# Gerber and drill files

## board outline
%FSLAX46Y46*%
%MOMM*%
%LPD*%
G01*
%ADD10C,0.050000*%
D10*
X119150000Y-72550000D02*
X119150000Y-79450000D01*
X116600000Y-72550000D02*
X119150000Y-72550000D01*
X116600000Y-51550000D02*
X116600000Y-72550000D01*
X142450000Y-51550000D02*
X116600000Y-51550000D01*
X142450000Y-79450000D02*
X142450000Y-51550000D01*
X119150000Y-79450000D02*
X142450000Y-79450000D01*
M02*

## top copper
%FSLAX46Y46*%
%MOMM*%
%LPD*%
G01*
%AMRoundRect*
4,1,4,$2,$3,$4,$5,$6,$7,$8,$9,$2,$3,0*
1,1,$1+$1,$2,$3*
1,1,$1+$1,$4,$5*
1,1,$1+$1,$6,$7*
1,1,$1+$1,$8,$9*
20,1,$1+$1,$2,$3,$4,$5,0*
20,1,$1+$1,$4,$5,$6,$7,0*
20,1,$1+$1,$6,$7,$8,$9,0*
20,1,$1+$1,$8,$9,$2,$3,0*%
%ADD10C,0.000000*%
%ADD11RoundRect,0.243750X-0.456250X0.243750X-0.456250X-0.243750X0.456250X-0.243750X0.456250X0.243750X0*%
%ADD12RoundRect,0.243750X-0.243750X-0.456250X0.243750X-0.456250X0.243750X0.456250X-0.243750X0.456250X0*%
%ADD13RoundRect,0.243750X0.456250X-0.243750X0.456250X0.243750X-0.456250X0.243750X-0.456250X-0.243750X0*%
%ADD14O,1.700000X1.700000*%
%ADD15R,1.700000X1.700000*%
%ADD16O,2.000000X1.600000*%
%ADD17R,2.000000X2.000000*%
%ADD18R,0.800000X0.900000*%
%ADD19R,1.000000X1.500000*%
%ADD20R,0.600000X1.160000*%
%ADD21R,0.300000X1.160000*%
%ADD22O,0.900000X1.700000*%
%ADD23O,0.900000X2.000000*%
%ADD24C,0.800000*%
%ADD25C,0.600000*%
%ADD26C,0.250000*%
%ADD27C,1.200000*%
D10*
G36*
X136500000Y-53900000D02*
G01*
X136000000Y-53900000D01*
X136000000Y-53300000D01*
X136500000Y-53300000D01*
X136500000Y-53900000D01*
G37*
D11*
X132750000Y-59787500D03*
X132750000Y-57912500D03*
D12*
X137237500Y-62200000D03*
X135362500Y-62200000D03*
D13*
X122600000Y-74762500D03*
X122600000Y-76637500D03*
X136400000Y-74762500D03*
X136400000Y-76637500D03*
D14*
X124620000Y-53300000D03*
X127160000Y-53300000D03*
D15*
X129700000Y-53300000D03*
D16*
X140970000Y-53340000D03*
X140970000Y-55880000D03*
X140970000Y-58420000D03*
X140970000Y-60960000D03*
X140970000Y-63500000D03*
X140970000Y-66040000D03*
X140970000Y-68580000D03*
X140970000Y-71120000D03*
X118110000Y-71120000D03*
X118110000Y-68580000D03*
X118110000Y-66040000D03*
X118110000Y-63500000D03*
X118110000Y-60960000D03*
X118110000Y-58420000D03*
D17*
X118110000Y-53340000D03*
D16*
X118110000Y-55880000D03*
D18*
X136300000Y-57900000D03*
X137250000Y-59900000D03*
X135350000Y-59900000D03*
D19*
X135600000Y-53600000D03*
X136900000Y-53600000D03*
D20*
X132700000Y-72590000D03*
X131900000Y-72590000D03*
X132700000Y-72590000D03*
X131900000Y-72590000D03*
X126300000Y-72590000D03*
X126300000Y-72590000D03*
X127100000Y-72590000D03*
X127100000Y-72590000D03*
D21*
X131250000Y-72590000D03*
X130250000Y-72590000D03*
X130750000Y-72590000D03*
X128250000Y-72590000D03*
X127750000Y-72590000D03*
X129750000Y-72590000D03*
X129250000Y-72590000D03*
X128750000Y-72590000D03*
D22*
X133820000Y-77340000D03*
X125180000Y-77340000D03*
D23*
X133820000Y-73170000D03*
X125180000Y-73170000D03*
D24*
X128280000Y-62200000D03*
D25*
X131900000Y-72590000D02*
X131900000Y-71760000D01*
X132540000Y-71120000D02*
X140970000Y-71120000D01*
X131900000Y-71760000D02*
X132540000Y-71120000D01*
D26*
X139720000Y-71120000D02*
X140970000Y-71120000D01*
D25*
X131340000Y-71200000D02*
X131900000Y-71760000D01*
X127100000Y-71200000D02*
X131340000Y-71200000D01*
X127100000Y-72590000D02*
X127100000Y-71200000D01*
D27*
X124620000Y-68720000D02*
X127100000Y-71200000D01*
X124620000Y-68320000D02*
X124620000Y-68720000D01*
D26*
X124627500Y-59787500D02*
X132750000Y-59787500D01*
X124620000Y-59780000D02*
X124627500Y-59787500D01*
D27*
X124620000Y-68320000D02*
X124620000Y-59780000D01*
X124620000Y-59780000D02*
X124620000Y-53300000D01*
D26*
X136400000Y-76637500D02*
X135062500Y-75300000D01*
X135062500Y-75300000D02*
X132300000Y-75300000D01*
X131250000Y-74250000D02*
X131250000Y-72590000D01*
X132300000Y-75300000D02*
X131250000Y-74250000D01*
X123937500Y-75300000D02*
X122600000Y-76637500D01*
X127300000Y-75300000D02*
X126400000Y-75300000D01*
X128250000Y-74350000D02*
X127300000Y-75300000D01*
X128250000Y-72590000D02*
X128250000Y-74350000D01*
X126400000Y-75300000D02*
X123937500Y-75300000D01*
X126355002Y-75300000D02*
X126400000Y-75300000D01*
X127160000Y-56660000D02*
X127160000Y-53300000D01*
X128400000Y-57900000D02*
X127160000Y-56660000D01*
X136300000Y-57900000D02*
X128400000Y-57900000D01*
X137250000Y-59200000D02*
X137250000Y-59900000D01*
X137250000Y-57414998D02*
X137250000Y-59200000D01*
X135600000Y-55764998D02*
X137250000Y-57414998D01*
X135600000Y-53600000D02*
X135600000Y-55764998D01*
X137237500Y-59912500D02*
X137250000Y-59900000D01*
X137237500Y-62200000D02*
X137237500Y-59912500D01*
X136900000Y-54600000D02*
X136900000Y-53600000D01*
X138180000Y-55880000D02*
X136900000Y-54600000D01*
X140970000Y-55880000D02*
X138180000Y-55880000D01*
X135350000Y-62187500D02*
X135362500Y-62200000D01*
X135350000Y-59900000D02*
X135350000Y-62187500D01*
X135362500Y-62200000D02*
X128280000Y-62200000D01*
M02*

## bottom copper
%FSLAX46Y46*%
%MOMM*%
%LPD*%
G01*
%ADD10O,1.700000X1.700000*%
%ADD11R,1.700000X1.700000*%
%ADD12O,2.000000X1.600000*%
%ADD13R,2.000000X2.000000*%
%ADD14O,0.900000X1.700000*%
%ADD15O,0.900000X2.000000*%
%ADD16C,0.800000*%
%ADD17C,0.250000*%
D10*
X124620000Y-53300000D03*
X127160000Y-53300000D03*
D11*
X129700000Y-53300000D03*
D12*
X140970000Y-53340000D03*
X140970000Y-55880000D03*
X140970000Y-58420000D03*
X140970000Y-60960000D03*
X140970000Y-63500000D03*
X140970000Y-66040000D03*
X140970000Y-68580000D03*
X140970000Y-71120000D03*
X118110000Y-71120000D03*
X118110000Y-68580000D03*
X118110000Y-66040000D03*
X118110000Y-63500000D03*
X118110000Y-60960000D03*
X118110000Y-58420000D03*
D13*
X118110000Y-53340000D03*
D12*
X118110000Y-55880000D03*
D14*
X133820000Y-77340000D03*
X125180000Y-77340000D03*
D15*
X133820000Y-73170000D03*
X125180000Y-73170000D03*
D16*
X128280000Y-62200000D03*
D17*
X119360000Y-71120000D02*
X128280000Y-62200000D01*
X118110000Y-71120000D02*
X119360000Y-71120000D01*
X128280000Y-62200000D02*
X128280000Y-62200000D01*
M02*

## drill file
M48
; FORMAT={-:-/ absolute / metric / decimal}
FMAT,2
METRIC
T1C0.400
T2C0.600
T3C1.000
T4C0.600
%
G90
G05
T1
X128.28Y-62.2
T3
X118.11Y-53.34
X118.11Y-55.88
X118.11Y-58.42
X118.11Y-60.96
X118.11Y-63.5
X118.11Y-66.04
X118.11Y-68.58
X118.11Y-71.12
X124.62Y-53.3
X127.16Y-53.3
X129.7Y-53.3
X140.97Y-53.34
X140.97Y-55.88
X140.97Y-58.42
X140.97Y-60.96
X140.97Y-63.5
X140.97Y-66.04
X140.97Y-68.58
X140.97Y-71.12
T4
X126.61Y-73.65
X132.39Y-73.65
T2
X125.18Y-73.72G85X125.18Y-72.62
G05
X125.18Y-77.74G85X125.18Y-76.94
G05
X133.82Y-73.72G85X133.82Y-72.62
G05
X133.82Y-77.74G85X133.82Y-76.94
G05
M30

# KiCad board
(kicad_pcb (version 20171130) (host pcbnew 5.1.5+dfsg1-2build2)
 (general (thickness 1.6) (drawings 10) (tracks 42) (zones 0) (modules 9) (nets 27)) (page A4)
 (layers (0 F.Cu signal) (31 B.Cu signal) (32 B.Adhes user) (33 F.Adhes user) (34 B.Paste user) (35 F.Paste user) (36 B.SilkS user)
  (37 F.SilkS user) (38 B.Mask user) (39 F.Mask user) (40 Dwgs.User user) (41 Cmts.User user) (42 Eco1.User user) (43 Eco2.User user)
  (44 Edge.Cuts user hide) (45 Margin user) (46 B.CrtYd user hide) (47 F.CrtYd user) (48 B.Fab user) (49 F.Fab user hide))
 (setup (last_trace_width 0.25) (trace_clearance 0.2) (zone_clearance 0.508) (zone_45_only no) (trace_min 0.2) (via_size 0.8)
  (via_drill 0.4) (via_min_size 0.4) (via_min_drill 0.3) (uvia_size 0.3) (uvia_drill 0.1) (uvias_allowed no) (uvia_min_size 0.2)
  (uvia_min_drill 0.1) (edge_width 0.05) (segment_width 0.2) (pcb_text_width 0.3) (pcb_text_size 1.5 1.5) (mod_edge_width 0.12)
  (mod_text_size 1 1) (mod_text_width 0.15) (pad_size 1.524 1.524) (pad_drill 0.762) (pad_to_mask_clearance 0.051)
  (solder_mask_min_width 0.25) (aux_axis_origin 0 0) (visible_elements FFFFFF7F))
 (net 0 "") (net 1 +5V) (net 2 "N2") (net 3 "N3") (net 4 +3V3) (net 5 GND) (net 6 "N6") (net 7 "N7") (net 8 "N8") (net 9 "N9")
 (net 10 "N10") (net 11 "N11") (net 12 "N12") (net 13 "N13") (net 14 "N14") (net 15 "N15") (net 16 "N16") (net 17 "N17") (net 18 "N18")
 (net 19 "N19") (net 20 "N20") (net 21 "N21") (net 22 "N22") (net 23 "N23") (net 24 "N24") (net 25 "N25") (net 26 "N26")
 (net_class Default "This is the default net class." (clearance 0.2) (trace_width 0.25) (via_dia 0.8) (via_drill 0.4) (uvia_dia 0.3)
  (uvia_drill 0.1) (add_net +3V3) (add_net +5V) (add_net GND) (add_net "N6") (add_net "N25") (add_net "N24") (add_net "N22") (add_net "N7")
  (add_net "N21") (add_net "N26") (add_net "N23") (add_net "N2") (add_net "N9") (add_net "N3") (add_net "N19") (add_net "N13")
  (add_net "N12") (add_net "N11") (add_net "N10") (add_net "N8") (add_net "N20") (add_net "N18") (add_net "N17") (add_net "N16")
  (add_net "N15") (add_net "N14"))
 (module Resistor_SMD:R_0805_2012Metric (layer F.Cu) (at 132.75 58.85 270)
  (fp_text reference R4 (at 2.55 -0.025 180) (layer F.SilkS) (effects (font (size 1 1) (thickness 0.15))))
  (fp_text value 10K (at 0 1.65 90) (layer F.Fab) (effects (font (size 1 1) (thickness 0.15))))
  (pad 2 smd roundrect (at 0.9375 0 270) (size 0.975 1.4) (layers F.Cu F.Paste F.Mask) (roundrect_rratio 0.25) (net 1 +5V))
  (pad 1 smd roundrect (at -0.9375 0 270) (size 0.975 1.4) (layers F.Cu F.Paste F.Mask) (roundrect_rratio 0.25) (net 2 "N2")))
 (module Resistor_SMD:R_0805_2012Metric (layer F.Cu) (at 136.3 62.2)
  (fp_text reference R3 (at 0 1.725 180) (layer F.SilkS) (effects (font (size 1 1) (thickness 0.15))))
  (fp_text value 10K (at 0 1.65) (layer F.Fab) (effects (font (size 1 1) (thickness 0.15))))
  (pad 2 smd roundrect (at 0.9375 0) (size 0.975 1.4) (layers F.Cu F.Paste F.Mask) (roundrect_rratio 0.25) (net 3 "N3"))
  (pad 1 smd roundrect (at -0.9375 0) (size 0.975 1.4) (layers F.Cu F.Paste F.Mask) (roundrect_rratio 0.25) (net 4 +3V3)))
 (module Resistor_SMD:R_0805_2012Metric (layer F.Cu) (at 122.6 75.7 90)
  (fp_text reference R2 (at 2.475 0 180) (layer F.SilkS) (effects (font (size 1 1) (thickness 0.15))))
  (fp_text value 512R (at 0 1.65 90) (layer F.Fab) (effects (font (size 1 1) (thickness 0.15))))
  (pad 2 smd roundrect (at 0.9375 0 90) (size 0.975 1.4) (layers F.Cu F.Paste F.Mask) (roundrect_rratio 0.25) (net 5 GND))
  (pad 1 smd roundrect (at -0.9375 0 90) (size 0.975 1.4) (layers F.Cu F.Paste F.Mask) (roundrect_rratio 0.25) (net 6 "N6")))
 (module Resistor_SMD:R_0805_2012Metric (layer F.Cu) (at 136.4 75.7 90)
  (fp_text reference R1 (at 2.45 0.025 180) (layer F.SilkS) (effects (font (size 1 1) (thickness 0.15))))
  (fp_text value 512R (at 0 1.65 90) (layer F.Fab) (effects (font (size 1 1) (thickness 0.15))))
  (pad 2 smd roundrect (at 0.9375 0 90) (size 0.975 1.4) (layers F.Cu F.Paste F.Mask) (roundrect_rratio 0.25) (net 5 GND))
  (pad 1 smd roundrect (at -0.9375 0 90) (size 0.975 1.4) (layers F.Cu F.Paste F.Mask) (roundrect_rratio 0.25) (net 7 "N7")))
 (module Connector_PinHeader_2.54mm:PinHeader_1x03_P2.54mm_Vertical (layer F.Cu) (at 129.7 53.3 270)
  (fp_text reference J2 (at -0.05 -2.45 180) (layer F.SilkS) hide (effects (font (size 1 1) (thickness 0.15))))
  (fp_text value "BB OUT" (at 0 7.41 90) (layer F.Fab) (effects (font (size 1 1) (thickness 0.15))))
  (pad 3 thru_hole oval (at 0 5.08 270) (size 1.7 1.7) (drill 1) (layers *.Cu *.Mask) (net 1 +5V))
  (pad 2 thru_hole oval (at 0 2.54 270) (size 1.7 1.7) (drill 1) (layers *.Cu *.Mask) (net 2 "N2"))
  (pad 1 thru_hole rect (at 0 0 270) (size 1.7 1.7) (drill 1) (layers *.Cu *.Mask) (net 5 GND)))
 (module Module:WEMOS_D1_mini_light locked (layer F.Cu) (at 118.11 53.34)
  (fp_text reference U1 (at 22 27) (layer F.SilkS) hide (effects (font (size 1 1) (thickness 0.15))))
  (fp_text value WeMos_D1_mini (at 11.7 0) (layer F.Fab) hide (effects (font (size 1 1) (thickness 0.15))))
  (pad 16 thru_hole oval (at 22.86 0) (size 2 1.6) (drill 1) (layers *.Cu *.Mask) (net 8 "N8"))
  (pad 15 thru_hole oval (at 22.86 2.54) (size 2 1.6) (drill 1) (layers *.Cu *.Mask) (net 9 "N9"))
  (pad 14 thru_hole oval (at 22.86 5.08) (size 2 1.6) (drill 1) (layers *.Cu *.Mask) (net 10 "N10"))
  (pad 13 thru_hole oval (at 22.86 7.62) (size 2 1.6) (drill 1) (layers *.Cu *.Mask) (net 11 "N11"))
  (pad 12 thru_hole oval (at 22.86 10.16) (size 2 1.6) (drill 1) (layers *.Cu *.Mask) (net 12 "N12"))
  (pad 11 thru_hole oval (at 22.86 12.7) (size 2 1.6) (drill 1) (layers *.Cu *.Mask) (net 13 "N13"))
  (pad 10 thru_hole oval (at 22.86 15.24) (size 2 1.6) (drill 1) (layers *.Cu *.Mask) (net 5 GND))
  (pad 9 thru_hole oval (at 22.86 17.78) (size 2 1.6) (drill 1) (layers *.Cu *.Mask) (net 1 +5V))
  (pad 8 thru_hole oval (at 0 17.78) (size 2 1.6) (drill 1) (layers *.Cu *.Mask) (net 4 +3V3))
  (pad 7 thru_hole oval (at 0 15.24) (size 2 1.6) (drill 1) (layers *.Cu *.Mask) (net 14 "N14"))
  (pad 6 thru_hole oval (at 0 12.7) (size 2 1.6) (drill 1) (layers *.Cu *.Mask) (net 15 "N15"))
  (pad 5 thru_hole oval (at 0 10.16) (size 2 1.6) (drill 1) (layers *.Cu *.Mask) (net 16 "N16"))
  (pad 4 thru_hole oval (at 0 7.62) (size 2 1.6) (drill 1) (layers *.Cu *.Mask) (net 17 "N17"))
  (pad 3 thru_hole oval (at 0 5.08) (size 2 1.6) (drill 1) (layers *.Cu *.Mask) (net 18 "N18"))
  (pad 1 thru_hole rect (at 0 0) (size 2 2) (drill 1) (layers *.Cu *.Mask) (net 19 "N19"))
  (pad 2 thru_hole oval (at 0 2.54) (size 2 1.6) (drill 1) (layers *.Cu *.Mask) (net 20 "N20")))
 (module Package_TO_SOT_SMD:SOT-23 (layer F.Cu) (at 136.3 58.9 90)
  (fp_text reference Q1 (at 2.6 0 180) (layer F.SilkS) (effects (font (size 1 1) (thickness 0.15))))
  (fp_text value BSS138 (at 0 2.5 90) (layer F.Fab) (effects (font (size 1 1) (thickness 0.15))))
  (pad 3 smd rect (at 1 0 90) (size 0.9 0.8) (layers F.Cu F.Paste F.Mask) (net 2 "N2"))
  (pad 2 smd rect (at -1 0.95 90) (size 0.9 0.8) (layers F.Cu F.Paste F.Mask) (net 3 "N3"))
  (pad 1 smd rect (at -1 -0.95 90) (size 0.9 0.8) (layers F.Cu F.Paste F.Mask) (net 4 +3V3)))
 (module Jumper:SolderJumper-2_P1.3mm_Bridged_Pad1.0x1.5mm (layer F.Cu) (at 136.25 53.6 180)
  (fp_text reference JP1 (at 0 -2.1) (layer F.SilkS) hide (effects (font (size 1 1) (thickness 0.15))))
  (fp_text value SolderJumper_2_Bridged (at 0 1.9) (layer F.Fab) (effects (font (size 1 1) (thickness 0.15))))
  (fp_poly (pts (xy -0.25 -0.3) (xy 0.25 -0.3) (xy 0.25 0.3) (xy -0.25 0.3)) (layer F.Cu) (width 0))
  (pad 2 smd rect (at 0.65 0 180) (size 1 1.5) (layers F.Cu F.Mask) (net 3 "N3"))
  (pad 1 smd rect (at -0.65 0 180) (size 1 1.5) (layers F.Cu F.Mask) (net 9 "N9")))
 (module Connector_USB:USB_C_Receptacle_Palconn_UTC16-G (layer F.Cu) (at 129.5 75.1)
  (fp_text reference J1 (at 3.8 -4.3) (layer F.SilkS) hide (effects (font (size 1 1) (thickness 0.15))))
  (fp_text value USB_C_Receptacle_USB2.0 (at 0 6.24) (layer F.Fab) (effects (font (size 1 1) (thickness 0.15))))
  (pad A12 smd rect (at 3.2 -2.51) (size 0.6 1.16) (layers F.Cu F.Paste F.Mask) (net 5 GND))
  (pad A9 smd rect (at 2.4 -2.51) (size 0.6 1.16) (layers F.Cu F.Paste F.Mask) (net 1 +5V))
  (pad B1 smd rect (at 3.2 -2.51) (size 0.6 1.16) (layers F.Cu F.Paste F.Mask) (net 5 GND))
  (pad B4 smd rect (at 2.4 -2.51) (size 0.6 1.16) (layers F.Cu F.Paste F.Mask) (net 1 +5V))
  (pad B12 smd rect (at -3.2 -2.51) (size 0.6 1.16) (layers F.Cu F.Paste F.Mask) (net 5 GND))
  (pad A1 smd rect (at -3.2 -2.51) (size 0.6 1.16) (layers F.Cu F.Paste F.Mask) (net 5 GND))
  (pad B9 smd rect (at -2.4 -2.51) (size 0.6 1.16) (layers F.Cu F.Paste F.Mask) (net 1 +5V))
  (pad A4 smd rect (at -2.4 -2.51) (size 0.6 1.16) (layers F.Cu F.Paste F.Mask) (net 1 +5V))
  (pad "" np_thru_hole circle (at -2.89 -1.45 180) (size 0.6 0.6) (drill 0.6) (layers *.Cu *.Mask))
  (pad "" np_thru_hole circle (at 2.89 -1.45 180) (size 0.6 0.6) (drill 0.6) (layers *.Cu *.Mask))
  (pad B5 smd rect (at 1.75 -2.51 180) (size 0.3 1.16) (layers F.Cu F.Paste F.Mask) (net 7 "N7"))
  (pad B6 smd rect (at 0.75 -2.51 180) (size 0.3 1.16) (layers F.Cu F.Paste F.Mask) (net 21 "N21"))
  (pad A8 smd rect (at 1.25 -2.51 180) (size 0.3 1.16) (layers F.Cu F.Paste F.Mask) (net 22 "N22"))
  (pad A5 smd rect (at -1.25 -2.51 180) (size 0.3 1.16) (layers F.Cu F.Paste F.Mask) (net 6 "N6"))
  (pad B8 smd rect (at -1.75 -2.51 180) (size 0.3 1.16) (layers F.Cu F.Paste F.Mask) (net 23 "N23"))
  (pad A7 smd rect (at 0.25 -2.51 180) (size 0.3 1.16) (layers F.Cu F.Paste F.Mask) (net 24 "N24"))
  (pad A6 smd rect (at -0.25 -2.51 180) (size 0.3 1.16) (layers F.Cu F.Paste F.Mask) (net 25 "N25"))
  (pad B7 smd rect (at -0.75 -2.51 180) (size 0.3 1.16) (layers F.Cu F.Paste F.Mask) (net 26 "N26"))
  (pad S1 thru_hole oval (at 4.32 2.24 90) (size 1.7 0.9) (drill oval 1.4 0.6) (layers *.Cu *.Mask) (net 5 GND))
  (pad S1 thru_hole oval (at -4.32 2.24 90) (size 1.7 0.9) (drill oval 1.4 0.6) (layers *.Cu *.Mask) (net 5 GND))
  (pad S1 thru_hole oval (at 4.32 -1.93 90) (size 2 0.9) (drill oval 1.7 0.6) (layers *.Cu *.Mask) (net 5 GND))
  (pad S1 thru_hole oval (at -4.32 -1.93 90) (size 2 0.9) (drill oval 1.7 0.6) (layers *.Cu *.Mask) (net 5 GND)))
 (gr_line (start 119.15 72.55) (end 119.15 79.45) (layer Edge.Cuts) (width 0.05))
 (gr_line (start 116.6 72.55) (end 119.15 72.55) (layer Edge.Cuts) (width 0.05))
 (gr_line (start 116.6 51.55) (end 116.6 72.55) (layer Edge.Cuts) (width 0.05))
 (gr_line (start 142.45 51.55) (end 116.6 51.55) (layer Edge.Cuts) (width 0.05))
 (gr_line (start 142.45 79.45) (end 142.45 51.55) (layer Edge.Cuts) (width 0.05))
 (gr_line (start 119.15 79.45) (end 142.45 79.45) (layer Edge.Cuts) (width 0.05))
 (segment (start 131.9 72.59) (end 131.9 71.76) (width 0.6) (layer F.Cu) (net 1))
 (segment (start 132.54 71.12) (end 140.97 71.12) (width 0.6) (layer F.Cu) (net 1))
 (segment (start 131.9 71.76) (end 132.54 71.12) (width 0.6) (layer F.Cu) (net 1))
 (segment (start 139.72 71.12) (end 140.97 71.12) (width 0.25) (layer F.Cu) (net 1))
 (segment (start 131.34 71.2) (end 131.9 71.76) (width 0.6) (layer F.Cu) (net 1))
 (segment (start 127.1 71.2) (end 131.34 71.2) (width 0.6) (layer F.Cu) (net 1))
 (segment (start 127.1 72.59) (end 127.1 71.2) (width 0.6) (layer F.Cu) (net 1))
 (segment (start 124.62 68.72) (end 127.1 71.2) (width 1.2) (layer F.Cu) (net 1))
 (segment (start 124.62 68.32) (end 124.62 68.72) (width 1.2) (layer F.Cu) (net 1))
 (segment (start 124.6275 59.7875) (end 132.75 59.7875) (width 0.25) (layer F.Cu) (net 1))
 (segment (start 124.62 59.78) (end 124.6275 59.7875) (width 0.25) (layer F.Cu) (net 1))
 (segment (start 124.62 68.32) (end 124.62 59.78) (width 1.2) (layer F.Cu) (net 1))
 (segment (start 124.62 59.78) (end 124.62 53.3) (width 1.2) (layer F.Cu) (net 1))
 (segment (start 136.4 76.6375) (end 135.0625 75.3) (width 0.25) (layer F.Cu) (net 7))
 (segment (start 135.0625 75.3) (end 132.3 75.3) (width 0.25) (layer F.Cu) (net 7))
 (segment (start 131.25 74.25) (end 131.25 72.59) (width 0.25) (layer F.Cu) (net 7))
 (segment (start 132.3 75.3) (end 131.25 74.25) (width 0.25) (layer F.Cu) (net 7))
 (segment (start 123.9375 75.3) (end 122.6 76.6375) (width 0.25) (layer F.Cu) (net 6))
 (segment (start 127.3 75.3) (end 126.4 75.3) (width 0.25) (layer F.Cu) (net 6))
 (segment (start 128.25 74.35) (end 127.3 75.3) (width 0.25) (layer F.Cu) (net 6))
 (segment (start 128.25 72.59) (end 128.25 74.35) (width 0.25) (layer F.Cu) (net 6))
 (segment (start 126.4 75.3) (end 123.9375 75.3) (width 0.25) (layer F.Cu) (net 6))
 (segment (start 126.355002 75.3) (end 126.4 75.3) (width 0.25) (layer F.Cu) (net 6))
 (segment (start 127.16 56.66) (end 127.16 53.3) (width 0.25) (layer F.Cu) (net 2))
 (segment (start 128.4 57.9) (end 127.16 56.66) (width 0.25) (layer F.Cu) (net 2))
 (segment (start 136.3 57.9) (end 128.4 57.9) (width 0.25) (layer F.Cu) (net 2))
 (segment (start 137.25 59.2) (end 137.25 59.9) (width 0.25) (layer F.Cu) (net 3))
 (segment (start 137.25 57.414998) (end 137.25 59.2) (width 0.25) (layer F.Cu) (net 3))
 (segment (start 135.6 55.764998) (end 137.25 57.414998) (width 0.25) (layer F.Cu) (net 3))
 (segment (start 135.6 53.6) (end 135.6 55.764998) (width 0.25) (layer F.Cu) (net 3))
 (segment (start 137.2375 59.9125) (end 137.25 59.9) (width 0.25) (layer F.Cu) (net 3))
 (segment (start 137.2375 62.2) (end 137.2375 59.9125) (width 0.25) (layer F.Cu) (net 3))
 (segment (start 136.9 54.6) (end 136.9 53.6) (width 0.25) (layer F.Cu) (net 9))
 (segment (start 138.18 55.88) (end 136.9 54.6) (width 0.25) (layer F.Cu) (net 9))
 (segment (start 140.97 55.88) (end 138.18 55.88) (width 0.25) (layer F.Cu) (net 9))
 (segment (start 135.35 62.1875) (end 135.3625 62.2) (width 0.25) (layer F.Cu) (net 4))
 (segment (start 135.35 59.9) (end 135.35 62.1875) (width 0.25) (layer F.Cu) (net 4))
 (segment (start 119.36 71.12) (end 128.28 62.2) (width 0.25) (layer B.Cu) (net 4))
 (segment (start 118.11 71.12) (end 119.36 71.12) (width 0.25) (layer B.Cu) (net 4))
 (segment (start 128.28 62.2) (end 128.28 62.2) (width 0.25) (layer B.Cu) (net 4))
 (via (at 128.28 62.2) (size 0.8) (drill 0.4) (layers F.Cu B.Cu) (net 4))
 (segment (start 135.3625 62.2) (end 128.28 62.2) (width 0.25) (layer F.Cu) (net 4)))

